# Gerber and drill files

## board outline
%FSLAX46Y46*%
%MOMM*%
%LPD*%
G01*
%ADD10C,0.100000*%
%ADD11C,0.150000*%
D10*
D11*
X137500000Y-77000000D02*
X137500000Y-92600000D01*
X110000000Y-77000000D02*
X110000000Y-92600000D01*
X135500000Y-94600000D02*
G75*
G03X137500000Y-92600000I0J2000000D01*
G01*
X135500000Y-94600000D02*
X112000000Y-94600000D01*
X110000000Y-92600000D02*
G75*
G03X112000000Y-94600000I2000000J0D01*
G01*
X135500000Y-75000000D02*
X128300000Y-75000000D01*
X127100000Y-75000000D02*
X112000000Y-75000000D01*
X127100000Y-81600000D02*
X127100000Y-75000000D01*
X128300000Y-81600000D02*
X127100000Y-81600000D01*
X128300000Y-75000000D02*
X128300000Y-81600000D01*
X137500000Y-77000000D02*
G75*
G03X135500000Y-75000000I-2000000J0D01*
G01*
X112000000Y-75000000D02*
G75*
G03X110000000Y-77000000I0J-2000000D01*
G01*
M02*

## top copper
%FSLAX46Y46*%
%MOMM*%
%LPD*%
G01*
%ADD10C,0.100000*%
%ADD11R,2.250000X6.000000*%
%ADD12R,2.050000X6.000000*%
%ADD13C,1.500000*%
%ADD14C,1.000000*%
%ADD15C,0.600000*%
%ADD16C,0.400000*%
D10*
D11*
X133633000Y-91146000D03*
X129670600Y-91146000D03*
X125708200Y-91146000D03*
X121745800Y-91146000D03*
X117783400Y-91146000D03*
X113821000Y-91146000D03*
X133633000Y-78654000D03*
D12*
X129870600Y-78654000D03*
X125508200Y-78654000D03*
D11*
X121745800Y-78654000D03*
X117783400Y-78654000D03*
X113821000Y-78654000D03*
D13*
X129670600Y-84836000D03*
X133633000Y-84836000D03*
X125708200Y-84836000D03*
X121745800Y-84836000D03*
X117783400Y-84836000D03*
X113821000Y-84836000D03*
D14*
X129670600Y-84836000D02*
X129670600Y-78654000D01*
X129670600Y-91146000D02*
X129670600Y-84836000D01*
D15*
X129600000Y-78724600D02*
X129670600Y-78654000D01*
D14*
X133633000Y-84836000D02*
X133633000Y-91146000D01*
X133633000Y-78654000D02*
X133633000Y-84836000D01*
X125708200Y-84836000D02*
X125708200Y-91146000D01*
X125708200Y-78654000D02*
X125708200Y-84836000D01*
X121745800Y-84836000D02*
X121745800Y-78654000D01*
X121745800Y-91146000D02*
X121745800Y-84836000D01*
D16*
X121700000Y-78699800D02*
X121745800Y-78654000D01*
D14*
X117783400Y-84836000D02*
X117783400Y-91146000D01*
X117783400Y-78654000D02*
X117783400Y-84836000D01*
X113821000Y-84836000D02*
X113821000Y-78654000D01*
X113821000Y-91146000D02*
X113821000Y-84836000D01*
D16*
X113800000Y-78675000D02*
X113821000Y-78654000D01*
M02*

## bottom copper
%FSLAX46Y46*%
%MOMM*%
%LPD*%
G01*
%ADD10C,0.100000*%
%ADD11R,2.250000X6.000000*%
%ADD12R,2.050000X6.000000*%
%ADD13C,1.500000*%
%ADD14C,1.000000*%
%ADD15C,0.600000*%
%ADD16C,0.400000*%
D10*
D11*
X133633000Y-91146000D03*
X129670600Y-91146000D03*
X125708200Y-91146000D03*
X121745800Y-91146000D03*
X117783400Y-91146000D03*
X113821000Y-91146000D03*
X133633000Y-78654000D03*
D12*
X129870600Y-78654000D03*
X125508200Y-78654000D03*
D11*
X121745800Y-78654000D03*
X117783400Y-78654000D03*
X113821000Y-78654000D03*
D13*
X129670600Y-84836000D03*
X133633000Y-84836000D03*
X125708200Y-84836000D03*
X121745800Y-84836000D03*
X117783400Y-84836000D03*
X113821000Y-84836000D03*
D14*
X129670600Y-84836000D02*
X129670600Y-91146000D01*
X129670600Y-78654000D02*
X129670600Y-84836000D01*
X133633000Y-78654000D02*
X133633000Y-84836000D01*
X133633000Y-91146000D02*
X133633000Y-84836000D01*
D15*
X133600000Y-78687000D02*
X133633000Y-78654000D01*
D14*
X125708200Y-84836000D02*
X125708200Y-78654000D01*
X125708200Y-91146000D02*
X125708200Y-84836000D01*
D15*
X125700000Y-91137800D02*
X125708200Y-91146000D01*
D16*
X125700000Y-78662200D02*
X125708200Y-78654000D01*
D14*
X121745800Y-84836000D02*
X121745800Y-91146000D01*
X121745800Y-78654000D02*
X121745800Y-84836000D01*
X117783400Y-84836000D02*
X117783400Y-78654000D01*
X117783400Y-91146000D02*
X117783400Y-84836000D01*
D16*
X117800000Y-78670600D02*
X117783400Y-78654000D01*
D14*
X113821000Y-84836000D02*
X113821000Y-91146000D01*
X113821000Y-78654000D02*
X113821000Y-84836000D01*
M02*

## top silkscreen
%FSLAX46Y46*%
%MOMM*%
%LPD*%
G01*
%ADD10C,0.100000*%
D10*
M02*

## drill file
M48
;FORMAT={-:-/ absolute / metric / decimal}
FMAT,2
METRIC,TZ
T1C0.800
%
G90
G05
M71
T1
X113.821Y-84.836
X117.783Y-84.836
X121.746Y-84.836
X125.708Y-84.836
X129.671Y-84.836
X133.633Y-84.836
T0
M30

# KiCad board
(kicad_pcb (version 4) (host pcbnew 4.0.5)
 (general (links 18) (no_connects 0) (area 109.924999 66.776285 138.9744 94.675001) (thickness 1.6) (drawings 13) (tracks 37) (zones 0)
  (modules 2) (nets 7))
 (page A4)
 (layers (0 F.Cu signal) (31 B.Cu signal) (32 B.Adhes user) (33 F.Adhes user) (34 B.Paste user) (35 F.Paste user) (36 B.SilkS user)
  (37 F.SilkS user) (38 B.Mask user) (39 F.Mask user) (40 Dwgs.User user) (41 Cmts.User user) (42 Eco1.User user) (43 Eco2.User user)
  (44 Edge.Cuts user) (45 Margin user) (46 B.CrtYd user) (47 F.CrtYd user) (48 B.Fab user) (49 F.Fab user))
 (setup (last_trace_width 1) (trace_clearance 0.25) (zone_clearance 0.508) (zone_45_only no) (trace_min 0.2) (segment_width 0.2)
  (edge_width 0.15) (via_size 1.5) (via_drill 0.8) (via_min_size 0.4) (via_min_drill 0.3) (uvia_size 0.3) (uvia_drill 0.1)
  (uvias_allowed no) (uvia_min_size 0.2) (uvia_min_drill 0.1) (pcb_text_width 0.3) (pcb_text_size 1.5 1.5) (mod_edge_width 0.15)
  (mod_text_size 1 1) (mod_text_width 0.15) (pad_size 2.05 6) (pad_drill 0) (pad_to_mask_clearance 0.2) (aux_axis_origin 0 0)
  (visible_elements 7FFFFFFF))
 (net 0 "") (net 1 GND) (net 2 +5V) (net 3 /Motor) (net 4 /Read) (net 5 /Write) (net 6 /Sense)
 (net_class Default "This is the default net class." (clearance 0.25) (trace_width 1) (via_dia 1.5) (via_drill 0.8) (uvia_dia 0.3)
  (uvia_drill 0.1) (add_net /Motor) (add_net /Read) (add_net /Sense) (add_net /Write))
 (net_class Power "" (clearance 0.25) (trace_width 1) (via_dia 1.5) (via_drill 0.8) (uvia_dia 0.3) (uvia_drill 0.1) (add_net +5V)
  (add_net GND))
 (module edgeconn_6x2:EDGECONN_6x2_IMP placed (layer F.Cu) (at 123.6 90.892 180)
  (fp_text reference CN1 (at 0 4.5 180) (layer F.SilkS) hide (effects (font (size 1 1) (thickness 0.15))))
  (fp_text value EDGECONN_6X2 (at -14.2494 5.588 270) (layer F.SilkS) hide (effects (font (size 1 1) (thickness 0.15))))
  (pad 1 smd rect (at -10.033 -0.254 180) (size 2.25 6) (layers F.Cu F.Paste F.Mask) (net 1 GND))
  (pad 2 smd rect (at -6.0706 -0.254 180) (size 2.25 6) (layers F.Cu F.Paste F.Mask) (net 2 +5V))
  (pad 3 smd rect (at -2.1082 -0.254 180) (size 2.25 6) (layers F.Cu F.Paste F.Mask) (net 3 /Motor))
  (pad 4 smd rect (at 1.8542 -0.254 180) (size 2.25 6) (layers F.Cu F.Paste F.Mask) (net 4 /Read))
  (pad 5 smd rect (at 5.8166 -0.254 180) (size 2.25 6) (layers F.Cu F.Paste F.Mask) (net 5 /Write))
  (pad 6 smd rect (at 9.779 -0.254 180) (size 2.25 6) (layers F.Cu F.Paste F.Mask) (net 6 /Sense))
  (pad A smd rect (at -10.033 -0.254 180) (size 2.25 6) (layers B.Cu B.Paste B.Mask) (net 1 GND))
  (pad B smd rect (at -6.0706 -0.254 180) (size 2.25 6) (layers B.Cu B.Paste B.Mask) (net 2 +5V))
  (pad C smd rect (at -2.1082 -0.254 180) (size 2.25 6) (layers B.Cu B.Paste B.Mask) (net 3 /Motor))
  (pad D smd rect (at 1.8542 -0.254 180) (size 2.25 6) (layers B.Cu B.Paste B.Mask) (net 4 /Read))
  (pad E smd rect (at 5.8166 -0.254 180) (size 2.25 6) (layers B.Cu B.Paste B.Mask) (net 5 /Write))
  (pad F smd rect (at 9.779 -0.254 180) (size 2.25 6) (layers B.Cu B.Paste B.Mask) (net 6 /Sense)))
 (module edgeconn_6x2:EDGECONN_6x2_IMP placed (layer F.Cu) (at 123.6 78.4 180)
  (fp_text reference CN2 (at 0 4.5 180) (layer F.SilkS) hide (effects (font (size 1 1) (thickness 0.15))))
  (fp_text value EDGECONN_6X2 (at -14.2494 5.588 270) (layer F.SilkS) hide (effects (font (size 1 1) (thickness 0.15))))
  (pad 1 smd rect (at -10.033 -0.254 180) (size 2.25 6) (layers F.Cu F.Paste F.Mask) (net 1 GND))
  (pad 2 smd rect (at -6.0706 -0.254 180) (size 2.05 6) (drill (offset -0.2 0)) (layers F.Cu F.Paste F.Mask) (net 2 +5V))
  (pad 3 smd rect (at -2.1082 -0.254 180) (size 2.05 6) (drill (offset 0.2 0)) (layers F.Cu F.Paste F.Mask) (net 3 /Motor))
  (pad 4 smd rect (at 1.8542 -0.254 180) (size 2.25 6) (layers F.Cu F.Paste F.Mask) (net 4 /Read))
  (pad 5 smd rect (at 5.8166 -0.254 180) (size 2.25 6) (layers F.Cu F.Paste F.Mask) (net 5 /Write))
  (pad 6 smd rect (at 9.779 -0.254 180) (size 2.25 6) (layers F.Cu F.Paste F.Mask) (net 6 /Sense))
  (pad A smd rect (at -10.033 -0.254 180) (size 2.25 6) (layers B.Cu B.Paste B.Mask) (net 1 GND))
  (pad B smd rect (at -6.0706 -0.254 180) (size 2.05 6) (drill (offset -0.2 0)) (layers B.Cu B.Paste B.Mask) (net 2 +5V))
  (pad C smd rect (at -2.1082 -0.254 180) (size 2.05 6) (drill (offset 0.2 0)) (layers B.Cu B.Paste B.Mask) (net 3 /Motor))
  (pad D smd rect (at 1.8542 -0.254 180) (size 2.25 6) (layers B.Cu B.Paste B.Mask) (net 4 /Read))
  (pad E smd rect (at 5.8166 -0.254 180) (size 2.25 6) (layers B.Cu B.Paste B.Mask) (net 5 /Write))
  (pad F smd rect (at 9.779 -0.254 180) (size 2.25 6) (layers B.Cu B.Paste B.Mask) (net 6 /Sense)))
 (gr_line (start 137.5 77) (end 137.5 92.6) (layer Edge.Cuts) (width 0.15))
 (gr_line (start 110 77) (end 110 92.6) (layer Edge.Cuts) (width 0.15))
 (gr_arc (start 135.5 92.6) (end 137.5 92.6) (angle 90) (layer Edge.Cuts) (width 0.15))
 (gr_line (start 135.5 94.6) (end 112 94.6) (layer Edge.Cuts) (width 0.15))
 (gr_arc (start 112 92.6) (end 112 94.6) (angle 90) (layer Edge.Cuts) (width 0.15))
 (gr_line (start 135.5 75) (end 128.3 75) (layer Edge.Cuts) (width 0.15))
 (gr_line (start 127.1 75) (end 112 75) (layer Edge.Cuts) (width 0.15))
 (gr_line (start 127.1 81.6) (end 127.1 75) (layer Edge.Cuts) (width 0.15))
 (gr_line (start 128.3 81.6) (end 127.1 81.6) (layer Edge.Cuts) (width 0.15))
 (gr_line (start 128.3 75) (end 128.3 81.6) (layer Edge.Cuts) (width 0.15))
 (gr_arc (start 135.5 77) (end 135.5 75) (angle 90) (layer Edge.Cuts) (width 0.15))
 (gr_arc (start 112 77) (end 110 77) (angle 90) (layer Edge.Cuts) (width 0.15))
 (segment (start 129.6706 84.836) (end 129.6706 91.146) (width 1) (layer B.Cu) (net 2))
 (segment (start 129.6706 78.654) (end 129.6706 84.836) (width 1) (layer B.Cu) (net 2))
 (segment (start 129.6706 84.836) (end 129.6706 78.654) (width 1) (layer F.Cu) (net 2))
 (segment (start 129.6706 91.146) (end 129.6706 84.836) (width 1) (layer F.Cu) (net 2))
 (via (at 129.6706 84.836) (size 1.5) (drill 0.8) (layers F.Cu B.Cu) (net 2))
 (segment (start 129.6 78.7246) (end 129.6706 78.654) (width 0.6) (layer F.Cu) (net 2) (status 30))
 (segment (start 133.633 78.654) (end 133.633 84.836) (width 1) (layer B.Cu) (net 1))
 (segment (start 133.633 91.146) (end 133.633 84.836) (width 1) (layer B.Cu) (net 1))
 (segment (start 133.633 84.836) (end 133.633 91.146) (width 1) (layer F.Cu) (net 1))
 (segment (start 133.633 78.654) (end 133.633 84.836) (width 1) (layer F.Cu) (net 1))
 (via (at 133.633 84.836) (size 1.5) (drill 0.8) (layers F.Cu B.Cu) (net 1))
 (segment (start 133.6 78.687) (end 133.633 78.654) (width 0.6) (layer B.Cu) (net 1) (status 30))
 (segment (start 125.7082 84.836) (end 125.7082 78.654) (width 1) (layer B.Cu) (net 3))
 (segment (start 125.7082 91.146) (end 125.7082 84.836) (width 1) (layer B.Cu) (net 3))
 (segment (start 125.7082 84.836) (end 125.7082 91.146) (width 1) (layer F.Cu) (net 3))
 (segment (start 125.7082 78.654) (end 125.7082 84.836) (width 1) (layer F.Cu) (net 3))
 (via (at 125.7082 84.836) (size 1.5) (drill 0.8) (layers F.Cu B.Cu) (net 3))
 (segment (start 125.7 91.1378) (end 125.7082 91.146) (width 0.6) (layer B.Cu) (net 3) (status 30))
 (segment (start 125.7 78.6622) (end 125.7082 78.654) (width 0.4) (layer B.Cu) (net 3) (status 30))
 (segment (start 121.7458 84.836) (end 121.7458 91.146) (width 1) (layer B.Cu) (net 4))
 (segment (start 121.7458 78.654) (end 121.7458 84.836) (width 1) (layer B.Cu) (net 4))
 (segment (start 121.7458 84.836) (end 121.7458 78.654) (width 1) (layer F.Cu) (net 4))
 (segment (start 121.7458 91.146) (end 121.7458 84.836) (width 1) (layer F.Cu) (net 4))
 (via (at 121.7458 84.836) (size 1.5) (drill 0.8) (layers F.Cu B.Cu) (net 4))
 (segment (start 121.7 78.6998) (end 121.7458 78.654) (width 0.4) (layer F.Cu) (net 4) (status 30))
 (segment (start 117.7834 84.836) (end 117.7834 78.654) (width 1) (layer B.Cu) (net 5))
 (segment (start 117.7834 91.146) (end 117.7834 84.836) (width 1) (layer B.Cu) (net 5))
 (segment (start 117.7834 84.836) (end 117.7834 91.146) (width 1) (layer F.Cu) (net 5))
 (segment (start 117.7834 78.654) (end 117.7834 84.836) (width 1) (layer F.Cu) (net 5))
 (via (at 117.7834 84.836) (size 1.5) (drill 0.8) (layers F.Cu B.Cu) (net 5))
 (segment (start 117.8 78.6706) (end 117.7834 78.654) (width 0.4) (layer B.Cu) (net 5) (status 30))
 (segment (start 113.821 84.836) (end 113.821 91.146) (width 1) (layer B.Cu) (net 6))
 (segment (start 113.821 78.654) (end 113.821 84.836) (width 1) (layer B.Cu) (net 6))
 (segment (start 113.821 84.836) (end 113.821 78.654) (width 1) (layer F.Cu) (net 6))
 (segment (start 113.821 91.146) (end 113.821 84.836) (width 1) (layer F.Cu) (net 6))
 (via (at 113.821 84.836) (size 1.5) (drill 0.8) (layers F.Cu B.Cu) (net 6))
 (segment (start 113.8 78.675) (end 113.821 78.654) (width 0.4) (layer F.Cu) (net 6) (status 30)))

